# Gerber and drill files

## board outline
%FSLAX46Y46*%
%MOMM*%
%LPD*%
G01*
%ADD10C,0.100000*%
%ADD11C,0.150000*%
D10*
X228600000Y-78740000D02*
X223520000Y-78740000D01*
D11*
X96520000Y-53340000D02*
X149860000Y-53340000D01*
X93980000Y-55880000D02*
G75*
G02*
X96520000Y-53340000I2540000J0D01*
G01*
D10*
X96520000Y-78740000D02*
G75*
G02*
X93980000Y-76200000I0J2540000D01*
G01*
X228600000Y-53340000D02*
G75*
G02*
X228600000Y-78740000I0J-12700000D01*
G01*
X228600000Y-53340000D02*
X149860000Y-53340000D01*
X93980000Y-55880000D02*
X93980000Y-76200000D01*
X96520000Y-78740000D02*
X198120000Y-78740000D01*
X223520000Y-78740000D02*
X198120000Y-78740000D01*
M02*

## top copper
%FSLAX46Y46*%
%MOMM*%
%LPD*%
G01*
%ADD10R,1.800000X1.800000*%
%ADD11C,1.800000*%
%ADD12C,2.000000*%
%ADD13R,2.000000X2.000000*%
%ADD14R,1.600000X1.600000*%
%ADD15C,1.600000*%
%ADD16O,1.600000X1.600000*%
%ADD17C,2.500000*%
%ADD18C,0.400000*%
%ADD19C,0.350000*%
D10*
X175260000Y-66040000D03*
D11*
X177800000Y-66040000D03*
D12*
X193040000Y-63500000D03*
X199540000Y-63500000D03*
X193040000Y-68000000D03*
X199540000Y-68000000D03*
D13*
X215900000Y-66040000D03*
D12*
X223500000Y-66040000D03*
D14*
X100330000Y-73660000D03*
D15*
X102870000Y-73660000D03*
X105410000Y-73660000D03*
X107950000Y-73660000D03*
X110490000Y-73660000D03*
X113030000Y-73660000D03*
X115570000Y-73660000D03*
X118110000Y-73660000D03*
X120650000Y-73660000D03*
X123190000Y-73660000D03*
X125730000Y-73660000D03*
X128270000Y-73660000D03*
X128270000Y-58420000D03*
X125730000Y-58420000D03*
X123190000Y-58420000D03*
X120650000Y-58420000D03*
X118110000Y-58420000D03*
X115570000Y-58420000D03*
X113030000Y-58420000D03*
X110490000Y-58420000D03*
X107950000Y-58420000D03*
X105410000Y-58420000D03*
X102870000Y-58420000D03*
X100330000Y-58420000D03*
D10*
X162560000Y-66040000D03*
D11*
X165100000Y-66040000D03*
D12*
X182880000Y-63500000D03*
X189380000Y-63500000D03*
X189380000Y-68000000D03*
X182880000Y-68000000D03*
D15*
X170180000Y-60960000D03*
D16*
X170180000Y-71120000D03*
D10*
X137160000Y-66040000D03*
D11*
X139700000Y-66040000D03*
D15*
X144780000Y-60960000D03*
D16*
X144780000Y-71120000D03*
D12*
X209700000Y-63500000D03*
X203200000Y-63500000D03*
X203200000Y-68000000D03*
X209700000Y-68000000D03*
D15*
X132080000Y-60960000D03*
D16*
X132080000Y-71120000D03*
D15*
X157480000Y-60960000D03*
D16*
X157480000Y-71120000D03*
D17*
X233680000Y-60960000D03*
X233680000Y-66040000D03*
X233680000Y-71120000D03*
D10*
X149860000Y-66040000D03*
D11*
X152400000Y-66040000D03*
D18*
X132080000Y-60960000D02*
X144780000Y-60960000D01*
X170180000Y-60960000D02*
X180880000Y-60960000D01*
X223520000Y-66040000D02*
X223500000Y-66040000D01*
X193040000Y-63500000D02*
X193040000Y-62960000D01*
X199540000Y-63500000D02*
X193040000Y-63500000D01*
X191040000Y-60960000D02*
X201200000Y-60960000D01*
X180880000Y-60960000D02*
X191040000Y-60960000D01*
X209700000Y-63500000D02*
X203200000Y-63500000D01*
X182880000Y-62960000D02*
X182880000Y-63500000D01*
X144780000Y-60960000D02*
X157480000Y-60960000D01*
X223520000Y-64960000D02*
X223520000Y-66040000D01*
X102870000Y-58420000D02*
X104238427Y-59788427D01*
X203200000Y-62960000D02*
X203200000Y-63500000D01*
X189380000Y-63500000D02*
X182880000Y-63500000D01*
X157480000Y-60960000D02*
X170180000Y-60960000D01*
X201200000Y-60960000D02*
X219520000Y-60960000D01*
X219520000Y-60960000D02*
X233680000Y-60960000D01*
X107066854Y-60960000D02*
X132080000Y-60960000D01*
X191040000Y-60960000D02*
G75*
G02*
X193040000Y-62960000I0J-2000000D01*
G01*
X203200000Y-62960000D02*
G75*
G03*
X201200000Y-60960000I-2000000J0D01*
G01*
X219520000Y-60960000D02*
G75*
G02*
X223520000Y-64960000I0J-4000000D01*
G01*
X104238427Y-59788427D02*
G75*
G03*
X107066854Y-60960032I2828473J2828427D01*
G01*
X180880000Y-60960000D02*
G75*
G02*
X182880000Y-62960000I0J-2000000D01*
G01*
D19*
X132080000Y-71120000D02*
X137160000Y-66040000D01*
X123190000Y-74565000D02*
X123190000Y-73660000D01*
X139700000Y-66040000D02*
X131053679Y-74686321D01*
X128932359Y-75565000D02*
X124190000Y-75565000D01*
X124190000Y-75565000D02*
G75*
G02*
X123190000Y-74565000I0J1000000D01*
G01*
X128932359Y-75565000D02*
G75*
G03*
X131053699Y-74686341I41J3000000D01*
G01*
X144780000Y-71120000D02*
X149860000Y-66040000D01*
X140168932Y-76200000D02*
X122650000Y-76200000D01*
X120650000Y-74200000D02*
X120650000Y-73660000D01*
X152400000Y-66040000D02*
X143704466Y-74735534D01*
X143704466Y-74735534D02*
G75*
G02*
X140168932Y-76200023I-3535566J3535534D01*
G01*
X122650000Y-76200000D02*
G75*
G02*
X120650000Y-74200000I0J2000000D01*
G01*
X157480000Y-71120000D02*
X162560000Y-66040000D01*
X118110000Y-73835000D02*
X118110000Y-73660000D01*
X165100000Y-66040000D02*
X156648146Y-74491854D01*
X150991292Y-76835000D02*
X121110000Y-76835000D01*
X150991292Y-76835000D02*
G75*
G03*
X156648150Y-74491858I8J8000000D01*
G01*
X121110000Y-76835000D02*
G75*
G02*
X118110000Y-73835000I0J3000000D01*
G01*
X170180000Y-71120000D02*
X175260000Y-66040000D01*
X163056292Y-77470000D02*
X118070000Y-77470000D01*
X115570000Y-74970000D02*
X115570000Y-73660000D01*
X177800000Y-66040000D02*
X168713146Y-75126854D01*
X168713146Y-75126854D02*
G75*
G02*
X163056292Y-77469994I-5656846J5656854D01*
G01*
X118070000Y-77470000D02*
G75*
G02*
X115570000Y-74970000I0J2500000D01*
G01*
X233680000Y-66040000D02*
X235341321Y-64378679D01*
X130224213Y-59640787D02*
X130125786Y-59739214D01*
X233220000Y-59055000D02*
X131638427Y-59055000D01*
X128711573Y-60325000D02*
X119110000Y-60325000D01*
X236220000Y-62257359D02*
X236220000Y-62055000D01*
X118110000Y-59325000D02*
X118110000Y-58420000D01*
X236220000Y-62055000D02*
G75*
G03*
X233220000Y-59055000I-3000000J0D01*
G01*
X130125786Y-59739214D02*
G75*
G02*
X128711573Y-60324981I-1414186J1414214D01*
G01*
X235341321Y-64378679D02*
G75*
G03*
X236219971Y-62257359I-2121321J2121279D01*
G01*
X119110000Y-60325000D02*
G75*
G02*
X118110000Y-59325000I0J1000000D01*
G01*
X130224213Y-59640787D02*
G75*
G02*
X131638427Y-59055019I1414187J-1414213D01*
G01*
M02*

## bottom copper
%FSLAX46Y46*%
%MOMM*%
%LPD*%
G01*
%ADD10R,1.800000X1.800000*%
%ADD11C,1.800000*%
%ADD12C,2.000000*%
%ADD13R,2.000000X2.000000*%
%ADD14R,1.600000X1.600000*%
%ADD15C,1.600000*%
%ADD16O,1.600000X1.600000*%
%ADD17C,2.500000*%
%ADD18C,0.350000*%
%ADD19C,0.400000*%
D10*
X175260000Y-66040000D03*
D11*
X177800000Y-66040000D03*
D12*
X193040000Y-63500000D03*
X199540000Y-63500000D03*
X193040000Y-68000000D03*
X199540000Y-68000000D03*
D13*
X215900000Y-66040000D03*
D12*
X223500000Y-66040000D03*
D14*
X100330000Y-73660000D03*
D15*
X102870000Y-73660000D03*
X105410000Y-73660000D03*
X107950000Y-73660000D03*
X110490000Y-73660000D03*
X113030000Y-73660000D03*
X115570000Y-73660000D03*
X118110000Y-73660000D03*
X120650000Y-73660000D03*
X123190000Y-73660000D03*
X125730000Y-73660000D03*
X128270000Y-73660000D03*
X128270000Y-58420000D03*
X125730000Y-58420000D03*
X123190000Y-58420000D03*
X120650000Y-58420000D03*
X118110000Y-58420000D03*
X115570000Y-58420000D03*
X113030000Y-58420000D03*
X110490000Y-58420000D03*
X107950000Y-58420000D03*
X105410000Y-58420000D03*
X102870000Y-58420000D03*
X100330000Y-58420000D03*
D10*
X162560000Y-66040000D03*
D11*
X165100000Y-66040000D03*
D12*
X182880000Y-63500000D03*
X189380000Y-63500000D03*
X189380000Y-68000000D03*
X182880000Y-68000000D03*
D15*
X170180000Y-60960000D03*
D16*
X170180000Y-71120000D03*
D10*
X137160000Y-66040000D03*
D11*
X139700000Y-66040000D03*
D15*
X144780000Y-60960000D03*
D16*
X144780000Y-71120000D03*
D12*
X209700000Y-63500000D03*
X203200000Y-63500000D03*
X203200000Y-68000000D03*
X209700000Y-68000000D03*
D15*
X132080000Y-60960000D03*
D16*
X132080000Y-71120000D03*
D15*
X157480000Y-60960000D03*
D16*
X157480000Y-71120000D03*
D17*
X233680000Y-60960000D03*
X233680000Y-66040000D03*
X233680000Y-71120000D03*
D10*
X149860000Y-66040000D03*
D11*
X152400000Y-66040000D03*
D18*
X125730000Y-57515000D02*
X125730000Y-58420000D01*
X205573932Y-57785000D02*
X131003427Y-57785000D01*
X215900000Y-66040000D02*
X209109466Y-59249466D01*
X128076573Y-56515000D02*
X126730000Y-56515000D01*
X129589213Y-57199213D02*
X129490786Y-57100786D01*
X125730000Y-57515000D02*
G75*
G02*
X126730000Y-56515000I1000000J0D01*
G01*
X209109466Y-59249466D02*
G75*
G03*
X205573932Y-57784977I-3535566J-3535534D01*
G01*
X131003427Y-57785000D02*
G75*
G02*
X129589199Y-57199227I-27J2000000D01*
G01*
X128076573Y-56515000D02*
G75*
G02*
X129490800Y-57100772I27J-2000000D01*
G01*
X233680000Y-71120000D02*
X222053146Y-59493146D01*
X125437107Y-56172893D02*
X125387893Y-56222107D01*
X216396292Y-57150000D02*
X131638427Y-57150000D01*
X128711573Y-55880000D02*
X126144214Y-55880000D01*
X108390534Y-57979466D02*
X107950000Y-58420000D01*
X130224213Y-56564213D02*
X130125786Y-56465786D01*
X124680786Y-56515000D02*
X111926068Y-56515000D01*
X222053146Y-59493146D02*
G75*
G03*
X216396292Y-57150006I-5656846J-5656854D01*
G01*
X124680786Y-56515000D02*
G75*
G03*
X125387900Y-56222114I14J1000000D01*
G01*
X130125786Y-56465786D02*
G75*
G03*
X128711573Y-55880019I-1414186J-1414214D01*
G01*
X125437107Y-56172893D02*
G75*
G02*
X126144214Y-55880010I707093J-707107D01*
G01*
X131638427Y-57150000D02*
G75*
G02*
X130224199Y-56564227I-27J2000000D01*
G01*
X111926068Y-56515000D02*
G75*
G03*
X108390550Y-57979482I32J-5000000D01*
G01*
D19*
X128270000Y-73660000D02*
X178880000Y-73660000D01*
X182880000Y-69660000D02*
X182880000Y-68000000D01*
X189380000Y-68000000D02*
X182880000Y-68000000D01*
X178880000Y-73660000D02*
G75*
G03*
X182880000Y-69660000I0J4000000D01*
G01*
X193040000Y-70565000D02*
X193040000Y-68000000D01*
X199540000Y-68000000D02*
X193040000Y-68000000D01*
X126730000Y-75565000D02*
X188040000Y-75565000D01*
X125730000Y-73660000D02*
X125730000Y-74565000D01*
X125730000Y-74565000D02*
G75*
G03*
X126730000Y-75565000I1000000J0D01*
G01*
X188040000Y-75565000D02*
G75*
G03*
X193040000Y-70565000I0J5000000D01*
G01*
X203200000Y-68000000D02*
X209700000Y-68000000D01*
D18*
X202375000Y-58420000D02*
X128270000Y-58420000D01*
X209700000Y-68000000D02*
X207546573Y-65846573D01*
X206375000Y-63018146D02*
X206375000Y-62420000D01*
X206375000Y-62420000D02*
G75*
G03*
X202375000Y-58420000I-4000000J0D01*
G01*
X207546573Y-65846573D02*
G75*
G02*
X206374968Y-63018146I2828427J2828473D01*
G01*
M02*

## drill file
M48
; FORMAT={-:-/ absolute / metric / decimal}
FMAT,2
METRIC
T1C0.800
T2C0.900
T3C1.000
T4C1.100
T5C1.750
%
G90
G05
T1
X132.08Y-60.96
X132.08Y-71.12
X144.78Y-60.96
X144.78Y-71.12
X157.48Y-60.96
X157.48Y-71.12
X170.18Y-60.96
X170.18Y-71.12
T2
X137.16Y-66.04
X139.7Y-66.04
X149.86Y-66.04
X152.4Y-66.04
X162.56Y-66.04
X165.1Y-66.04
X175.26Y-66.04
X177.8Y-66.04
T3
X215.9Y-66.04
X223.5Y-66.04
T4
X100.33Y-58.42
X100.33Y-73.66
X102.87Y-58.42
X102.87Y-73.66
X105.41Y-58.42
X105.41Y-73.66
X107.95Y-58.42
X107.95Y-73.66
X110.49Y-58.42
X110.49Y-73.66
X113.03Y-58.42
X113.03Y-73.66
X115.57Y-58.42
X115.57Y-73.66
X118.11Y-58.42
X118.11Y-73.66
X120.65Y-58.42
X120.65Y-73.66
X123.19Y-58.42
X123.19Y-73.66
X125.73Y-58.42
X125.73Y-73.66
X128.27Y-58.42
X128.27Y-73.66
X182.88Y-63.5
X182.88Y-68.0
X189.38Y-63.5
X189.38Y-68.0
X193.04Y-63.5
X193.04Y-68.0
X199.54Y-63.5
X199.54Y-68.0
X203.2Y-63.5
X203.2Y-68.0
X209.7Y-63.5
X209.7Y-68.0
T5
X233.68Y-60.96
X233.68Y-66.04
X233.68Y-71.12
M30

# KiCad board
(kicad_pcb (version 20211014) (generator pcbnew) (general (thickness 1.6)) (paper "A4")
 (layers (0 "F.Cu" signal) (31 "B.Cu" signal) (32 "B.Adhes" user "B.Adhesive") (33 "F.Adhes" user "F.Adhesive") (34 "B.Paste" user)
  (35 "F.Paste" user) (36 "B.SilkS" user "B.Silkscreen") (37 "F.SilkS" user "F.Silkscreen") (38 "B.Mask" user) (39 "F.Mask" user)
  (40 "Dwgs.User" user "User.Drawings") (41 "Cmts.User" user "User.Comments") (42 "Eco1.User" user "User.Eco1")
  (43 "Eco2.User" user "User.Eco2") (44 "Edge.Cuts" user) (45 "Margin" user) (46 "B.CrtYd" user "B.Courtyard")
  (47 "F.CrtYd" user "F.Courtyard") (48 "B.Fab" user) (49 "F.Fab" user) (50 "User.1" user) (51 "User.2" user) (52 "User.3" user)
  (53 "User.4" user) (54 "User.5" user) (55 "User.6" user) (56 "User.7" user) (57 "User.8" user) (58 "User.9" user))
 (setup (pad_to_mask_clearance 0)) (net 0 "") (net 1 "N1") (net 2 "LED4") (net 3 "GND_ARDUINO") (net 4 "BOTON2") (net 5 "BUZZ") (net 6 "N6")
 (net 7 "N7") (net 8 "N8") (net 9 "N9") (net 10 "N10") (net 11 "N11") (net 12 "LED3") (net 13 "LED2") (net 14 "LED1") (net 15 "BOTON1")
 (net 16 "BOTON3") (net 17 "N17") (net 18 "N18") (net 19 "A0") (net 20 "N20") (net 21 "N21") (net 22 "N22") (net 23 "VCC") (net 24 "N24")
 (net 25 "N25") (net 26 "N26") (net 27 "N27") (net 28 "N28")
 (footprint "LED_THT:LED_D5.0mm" (layer "F.Cu") (at 175.26 66.04)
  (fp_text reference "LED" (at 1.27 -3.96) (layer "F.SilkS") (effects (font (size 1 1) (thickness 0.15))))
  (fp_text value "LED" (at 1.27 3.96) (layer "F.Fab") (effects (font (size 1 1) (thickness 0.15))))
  (pad "1" thru_hole rect (at 0 0) (size 1.8 1.8) (drill 0.9) (layers *.Cu *.Mask) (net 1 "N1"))
  (pad "2" thru_hole circle (at 2.54 0) (size 1.8 1.8) (drill 0.9) (layers *.Cu *.Mask) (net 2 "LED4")))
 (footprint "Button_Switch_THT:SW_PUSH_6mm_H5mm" (layer "F.Cu") (at 193.04 63.5)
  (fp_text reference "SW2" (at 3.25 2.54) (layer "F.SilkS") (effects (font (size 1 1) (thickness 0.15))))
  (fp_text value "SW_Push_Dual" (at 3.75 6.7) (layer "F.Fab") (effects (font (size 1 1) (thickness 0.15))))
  (pad "1" thru_hole circle (at 0 0 90) (size 2 2) (drill 1.1) (layers *.Cu *.Mask) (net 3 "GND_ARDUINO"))
  (pad "1" thru_hole circle (at 6.5 0 90) (size 2 2) (drill 1.1) (layers *.Cu *.Mask) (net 3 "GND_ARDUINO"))
  (pad "2" thru_hole circle (at 0 4.5 90) (size 2 2) (drill 1.1) (layers *.Cu *.Mask) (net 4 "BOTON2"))
  (pad "2" thru_hole circle (at 6.5 4.5 90) (size 2 2) (drill 1.1) (layers *.Cu *.Mask) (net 4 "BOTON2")))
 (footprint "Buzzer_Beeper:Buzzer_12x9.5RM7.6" (layer "F.Cu") (at 215.9 66.04)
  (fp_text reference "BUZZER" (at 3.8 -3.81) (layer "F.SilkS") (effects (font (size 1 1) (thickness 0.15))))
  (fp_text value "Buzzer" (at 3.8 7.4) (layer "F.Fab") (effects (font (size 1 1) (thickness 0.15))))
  (pad "1" thru_hole rect (at 0 0) (size 2 2) (drill 1) (layers *.Cu *.Mask) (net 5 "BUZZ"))
  (pad "2" thru_hole circle (at 7.6 0) (size 2 2) (drill 1) (layers *.Cu *.Mask) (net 3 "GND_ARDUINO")))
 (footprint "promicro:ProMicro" (layer "F.Cu") (at 114.3 66.04)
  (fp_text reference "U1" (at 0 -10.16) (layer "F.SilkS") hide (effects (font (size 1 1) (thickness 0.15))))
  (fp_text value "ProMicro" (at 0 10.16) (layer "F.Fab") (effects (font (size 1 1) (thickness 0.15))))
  (pad "1" thru_hole rect locked (at -13.97 7.62) (size 1.6 1.6) (drill 1.1) (layers *.Cu *.Mask "F.SilkS") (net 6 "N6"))
  (pad "2" thru_hole circle locked (at -11.43 7.62) (size 1.6 1.6) (drill 1.1) (layers *.Cu *.Mask "F.SilkS") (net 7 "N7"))
  (pad "3" thru_hole circle locked (at -8.89 7.62) (size 1.6 1.6) (drill 1.1) (layers *.Cu *.Mask "F.SilkS") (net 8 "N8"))
  (pad "4" thru_hole circle locked (at -6.35 7.62) (size 1.6 1.6) (drill 1.1) (layers *.Cu *.Mask "F.SilkS") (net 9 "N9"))
  (pad "5" thru_hole circle locked (at -3.81 7.62) (size 1.6 1.6) (drill 1.1) (layers *.Cu *.Mask "F.SilkS") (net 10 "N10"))
  (pad "6" thru_hole circle locked (at -1.27 7.62) (size 1.6 1.6) (drill 1.1) (layers *.Cu *.Mask "F.SilkS") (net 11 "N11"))
  (pad "7" thru_hole circle locked (at 1.27 7.62) (size 1.6 1.6) (drill 1.1) (layers *.Cu *.Mask "F.SilkS") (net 2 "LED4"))
  (pad "8" thru_hole circle locked (at 3.81 7.62) (size 1.6 1.6) (drill 1.1) (layers *.Cu *.Mask "F.SilkS") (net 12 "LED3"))
  (pad "9" thru_hole circle locked (at 6.35 7.62) (size 1.6 1.6) (drill 1.1) (layers *.Cu *.Mask "F.SilkS") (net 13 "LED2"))
  (pad "10" thru_hole circle locked (at 8.89 7.62) (size 1.6 1.6) (drill 1.1) (layers *.Cu *.Mask "F.SilkS") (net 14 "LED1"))
  (pad "11" thru_hole circle locked (at 11.43 7.62) (size 1.6 1.6) (drill 1.1) (layers *.Cu *.Mask "F.SilkS") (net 4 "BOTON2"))
  (pad "12" thru_hole circle locked (at 13.97 7.62) (size 1.6 1.6) (drill 1.1) (layers *.Cu *.Mask "F.SilkS") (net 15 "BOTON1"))
  (pad "13" thru_hole circle locked (at 13.97 -7.62) (size 1.6 1.6) (drill 1.1) (layers *.Cu *.Mask "F.SilkS") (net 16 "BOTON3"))
  (pad "14" thru_hole circle locked (at 11.43 -7.62) (size 1.6 1.6) (drill 1.1) (layers *.Cu *.Mask "F.SilkS") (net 5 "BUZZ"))
  (pad "15" thru_hole circle locked (at 8.89 -7.62) (size 1.6 1.6) (drill 1.1) (layers *.Cu *.Mask "F.SilkS") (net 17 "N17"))
  (pad "16" thru_hole circle locked (at 6.35 -7.62) (size 1.6 1.6) (drill 1.1) (layers *.Cu *.Mask "F.SilkS") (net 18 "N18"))
  (pad "17" thru_hole circle locked (at 3.81 -7.62) (size 1.6 1.6) (drill 1.1) (layers *.Cu *.Mask "F.SilkS") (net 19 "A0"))
  (pad "18" thru_hole circle locked (at 1.27 -7.62) (size 1.6 1.6) (drill 1.1) (layers *.Cu *.Mask "F.SilkS") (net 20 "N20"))
  (pad "19" thru_hole circle locked (at -1.27 -7.62) (size 1.6 1.6) (drill 1.1) (layers *.Cu *.Mask "F.SilkS") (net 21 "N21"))
  (pad "20" thru_hole circle locked (at -3.81 -7.62) (size 1.6 1.6) (drill 1.1) (layers *.Cu *.Mask "F.SilkS") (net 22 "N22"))
  (pad "21" thru_hole circle locked (at -6.35 -7.62) (size 1.6 1.6) (drill 1.1) (layers *.Cu *.Mask "F.SilkS") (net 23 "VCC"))
  (pad "22" thru_hole circle locked (at -8.89 -7.62) (size 1.6 1.6) (drill 1.1) (layers *.Cu *.Mask "F.SilkS") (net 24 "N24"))
  (pad "23" thru_hole circle locked (at -11.43 -7.62) (size 1.6 1.6) (drill 1.1) (layers *.Cu *.Mask "F.SilkS") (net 3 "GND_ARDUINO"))
  (pad "24" thru_hole circle locked (at -13.97 -7.62) (size 1.6 1.6) (drill 1.1) (layers *.Cu *.Mask "F.SilkS") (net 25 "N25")))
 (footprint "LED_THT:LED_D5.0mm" (layer "F.Cu") (at 162.56 66.04)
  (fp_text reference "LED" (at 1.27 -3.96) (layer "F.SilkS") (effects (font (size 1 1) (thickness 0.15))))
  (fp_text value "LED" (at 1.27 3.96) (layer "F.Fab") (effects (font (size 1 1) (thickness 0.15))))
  (pad "1" thru_hole rect (at 0 0) (size 1.8 1.8) (drill 0.9) (layers *.Cu *.Mask) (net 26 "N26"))
  (pad "2" thru_hole circle (at 2.54 0) (size 1.8 1.8) (drill 0.9) (layers *.Cu *.Mask) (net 12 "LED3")))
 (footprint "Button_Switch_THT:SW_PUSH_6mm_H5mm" (layer "F.Cu") (at 182.88 63.5)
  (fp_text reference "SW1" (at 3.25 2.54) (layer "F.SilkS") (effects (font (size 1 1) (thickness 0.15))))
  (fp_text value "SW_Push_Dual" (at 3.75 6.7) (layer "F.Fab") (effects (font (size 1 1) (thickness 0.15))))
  (pad "1" thru_hole circle (at 0 0 90) (size 2 2) (drill 1.1) (layers *.Cu *.Mask) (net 3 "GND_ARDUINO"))
  (pad "1" thru_hole circle (at 6.5 0 90) (size 2 2) (drill 1.1) (layers *.Cu *.Mask) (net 3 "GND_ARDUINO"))
  (pad "2" thru_hole circle (at 6.5 4.5 90) (size 2 2) (drill 1.1) (layers *.Cu *.Mask) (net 15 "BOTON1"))
  (pad "2" thru_hole circle (at 0 4.5 90) (size 2 2) (drill 1.1) (layers *.Cu *.Mask) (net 15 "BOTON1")))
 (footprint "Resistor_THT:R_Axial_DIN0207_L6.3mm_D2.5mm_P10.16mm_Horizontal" (layer "F.Cu") (at 170.18 60.96 -90)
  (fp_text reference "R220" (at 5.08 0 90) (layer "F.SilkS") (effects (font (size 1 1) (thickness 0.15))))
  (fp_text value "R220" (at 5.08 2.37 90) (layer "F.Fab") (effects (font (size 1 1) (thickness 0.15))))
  (pad "1" thru_hole circle (at 0 0 270) (size 1.6 1.6) (drill 0.8) (layers *.Cu *.Mask) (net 3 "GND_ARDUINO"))
  (pad "2" thru_hole oval (at 10.16 0 270) (size 1.6 1.6) (drill 0.8) (layers *.Cu *.Mask) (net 1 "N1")))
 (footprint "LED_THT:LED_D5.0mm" (layer "F.Cu") (at 137.16 66.04)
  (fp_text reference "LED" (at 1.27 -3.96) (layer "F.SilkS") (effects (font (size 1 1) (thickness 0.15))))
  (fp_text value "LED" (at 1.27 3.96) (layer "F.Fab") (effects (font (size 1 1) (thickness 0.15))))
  (pad "1" thru_hole rect (at 0 0) (size 1.8 1.8) (drill 0.9) (layers *.Cu *.Mask) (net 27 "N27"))
  (pad "2" thru_hole circle (at 2.54 0) (size 1.8 1.8) (drill 0.9) (layers *.Cu *.Mask) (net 14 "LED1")))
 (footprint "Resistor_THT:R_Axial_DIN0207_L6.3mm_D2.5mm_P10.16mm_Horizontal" (layer "F.Cu") (at 144.78 60.96 -90)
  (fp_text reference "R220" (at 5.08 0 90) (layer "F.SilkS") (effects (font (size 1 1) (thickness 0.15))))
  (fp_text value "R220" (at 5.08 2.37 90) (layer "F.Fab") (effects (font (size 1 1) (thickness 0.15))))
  (pad "1" thru_hole circle (at 0 0 270) (size 1.6 1.6) (drill 0.8) (layers *.Cu *.Mask) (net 3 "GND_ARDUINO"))
  (pad "2" thru_hole oval (at 10.16 0 270) (size 1.6 1.6) (drill 0.8) (layers *.Cu *.Mask) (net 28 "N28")))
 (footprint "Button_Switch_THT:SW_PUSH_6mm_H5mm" (layer "F.Cu") (at 203.2 63.5)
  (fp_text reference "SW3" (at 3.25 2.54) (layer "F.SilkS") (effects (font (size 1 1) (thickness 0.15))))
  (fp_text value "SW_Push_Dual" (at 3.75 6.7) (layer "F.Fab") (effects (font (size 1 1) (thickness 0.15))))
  (pad "1" thru_hole circle (at 6.5 0 90) (size 2 2) (drill 1.1) (layers *.Cu *.Mask) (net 3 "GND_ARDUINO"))
  (pad "1" thru_hole circle (at 0 0 90) (size 2 2) (drill 1.1) (layers *.Cu *.Mask) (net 3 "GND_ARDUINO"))
  (pad "2" thru_hole circle (at 0 4.5 90) (size 2 2) (drill 1.1) (layers *.Cu *.Mask) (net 16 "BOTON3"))
  (pad "2" thru_hole circle (at 6.5 4.5 90) (size 2 2) (drill 1.1) (layers *.Cu *.Mask) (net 16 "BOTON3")))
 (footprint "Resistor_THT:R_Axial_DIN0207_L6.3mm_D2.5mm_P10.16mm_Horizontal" (layer "F.Cu") (at 132.08 60.96 -90)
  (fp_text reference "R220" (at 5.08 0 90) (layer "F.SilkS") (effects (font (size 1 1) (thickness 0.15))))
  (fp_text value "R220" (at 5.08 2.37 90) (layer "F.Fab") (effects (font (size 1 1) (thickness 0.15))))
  (pad "1" thru_hole circle (at 0 0 270) (size 1.6 1.6) (drill 0.8) (layers *.Cu *.Mask) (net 3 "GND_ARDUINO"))
  (pad "2" thru_hole oval (at 10.16 0 270) (size 1.6 1.6) (drill 0.8) (layers *.Cu *.Mask) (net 27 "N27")))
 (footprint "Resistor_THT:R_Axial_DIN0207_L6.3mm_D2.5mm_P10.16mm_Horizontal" (layer "F.Cu") (at 157.48 60.96 -90)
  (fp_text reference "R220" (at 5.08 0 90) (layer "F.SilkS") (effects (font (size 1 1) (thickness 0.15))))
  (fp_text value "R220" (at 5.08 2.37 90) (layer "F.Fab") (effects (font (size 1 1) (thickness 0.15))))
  (pad "1" thru_hole circle (at 0 0 270) (size 1.6 1.6) (drill 0.8) (layers *.Cu *.Mask) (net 3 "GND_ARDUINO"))
  (pad "2" thru_hole oval (at 10.16 0 270) (size 1.6 1.6) (drill 0.8) (layers *.Cu *.Mask) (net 26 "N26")))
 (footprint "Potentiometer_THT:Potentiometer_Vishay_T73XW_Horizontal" (layer "F.Cu") (at 233.68 63.5)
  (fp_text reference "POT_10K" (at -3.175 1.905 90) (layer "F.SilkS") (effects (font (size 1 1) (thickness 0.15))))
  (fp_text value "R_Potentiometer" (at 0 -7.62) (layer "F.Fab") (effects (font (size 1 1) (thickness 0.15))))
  (pad "1" thru_hole circle (at 0 -2.54) (size 2.5 2.5) (drill 1.75) (layers *.Cu *.Mask) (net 3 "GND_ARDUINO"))
  (pad "2" thru_hole circle (at 0 2.54) (size 2.5 2.5) (drill 1.75) (layers *.Cu *.Mask) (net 19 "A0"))
  (pad "3" thru_hole circle (at 0 7.62) (size 2.5 2.5) (drill 1.75) (layers *.Cu *.Mask) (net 23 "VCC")))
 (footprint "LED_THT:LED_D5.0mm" (layer "F.Cu") (at 149.86 66.04)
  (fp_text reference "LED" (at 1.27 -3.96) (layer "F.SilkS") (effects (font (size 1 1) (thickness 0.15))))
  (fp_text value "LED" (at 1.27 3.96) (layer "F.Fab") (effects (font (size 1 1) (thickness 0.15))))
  (pad "1" thru_hole rect (at 0 0) (size 1.8 1.8) (drill 0.9) (layers *.Cu *.Mask) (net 28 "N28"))
  (pad "2" thru_hole circle (at 2.54 0) (size 1.8 1.8) (drill 0.9) (layers *.Cu *.Mask) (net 13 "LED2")))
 (gr_line (start 228.6 78.74) (end 223.52 78.74) (layer "Edge.Cuts") (width 0.1))
 (gr_line (start 96.52 53.34) (end 149.86 53.34) (layer "Edge.Cuts") (width 0.15))
 (gr_arc (start 93.98 55.88) (mid 94.723949 54.083949) (end 96.52 53.34) (layer "Edge.Cuts") (width 0.15))
 (gr_arc (start 96.52 78.74) (mid 94.723949 77.996051) (end 93.98 76.2) (layer "Edge.Cuts") (width 0.1))
 (gr_arc (start 228.6 53.34) (mid 241.3 66.04) (end 228.6 78.74) (layer "Edge.Cuts") (width 0.1))
 (gr_line (start 228.6 53.34) (end 149.86 53.34) (layer "Edge.Cuts") (width 0.1))
 (gr_line (start 93.98 55.88) (end 93.98 76.2) (layer "Edge.Cuts") (width 0.1))
 (gr_line (start 96.52 78.74) (end 198.12 78.74) (layer "Edge.Cuts") (width 0.1))
 (gr_line (start 223.52 78.74) (end 198.12 78.74) (layer "Edge.Cuts") (width 0.1))
 (segment (start 125.73 57.515) (end 125.73 58.42) (width 0.35) (layer "B.Cu") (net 5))
 (segment (start 205.573932 57.785) (end 131.003427 57.785) (width 0.35) (layer "B.Cu") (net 5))
 (segment (start 215.9 66.04) (end 209.109466 59.249466) (width 0.35) (layer "B.Cu") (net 5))
 (segment (start 128.076573 56.515) (end 126.73 56.515) (width 0.35) (layer "B.Cu") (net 5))
 (segment (start 129.589213 57.199213) (end 129.490786 57.100786) (width 0.35) (layer "B.Cu") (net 5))
 (arc (start 125.73 57.515) (mid 126.022893 56.807893) (end 126.73 56.515) (width 0.35) (layer "B.Cu") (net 5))
 (arc (start 209.109466 59.249466) (mid 207.487349 58.165602) (end 205.573932 57.785) (width 0.35) (layer "B.Cu") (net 5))
 (arc (start 131.003427 57.785) (mid 130.23806 57.632759) (end 129.589213 57.199213) (width 0.35) (layer "B.Cu") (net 5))
 (arc (start 128.076573 56.515) (mid 128.84194 56.667241) (end 129.490786 57.100786) (width 0.35) (layer "B.Cu") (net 5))
 (segment (start 132.08 60.96) (end 144.78 60.96) (width 0.4) (layer "F.Cu") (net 3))
 (segment (start 170.18 60.96) (end 180.88 60.96) (width 0.4) (layer "F.Cu") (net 3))
 (segment (start 223.52 66.04) (end 223.5 66.04) (width 0.4) (layer "F.Cu") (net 3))
 (segment (start 193.04 63.5) (end 193.04 62.96) (width 0.4) (layer "F.Cu") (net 3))
 (segment (start 199.54 63.5) (end 193.04 63.5) (width 0.4) (layer "F.Cu") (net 3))
 (segment (start 191.04 60.96) (end 201.2 60.96) (width 0.4) (layer "F.Cu") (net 3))
 (segment (start 180.88 60.96) (end 191.04 60.96) (width 0.4) (layer "F.Cu") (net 3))
 (segment (start 209.7 63.5) (end 203.2 63.5) (width 0.4) (layer "F.Cu") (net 3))
 (segment (start 182.88 62.96) (end 182.88 63.5) (width 0.4) (layer "F.Cu") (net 3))
 (segment (start 144.78 60.96) (end 157.48 60.96) (width 0.4) (layer "F.Cu") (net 3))
 (segment (start 223.52 64.96) (end 223.52 66.04) (width 0.4) (layer "F.Cu") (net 3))
 (segment (start 102.87 58.42) (end 104.238427 59.788427) (width 0.4) (layer "F.Cu") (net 3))
 (segment (start 203.2 62.96) (end 203.2 63.5) (width 0.4) (layer "F.Cu") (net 3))
 (segment (start 189.38 63.5) (end 182.88 63.5) (width 0.4) (layer "F.Cu") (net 3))
 (segment (start 157.48 60.96) (end 170.18 60.96) (width 0.4) (layer "F.Cu") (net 3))
 (segment (start 201.2 60.96) (end 219.52 60.96) (width 0.4) (layer "F.Cu") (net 3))
 (segment (start 219.52 60.96) (end 233.68 60.96) (width 0.4) (layer "F.Cu") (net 3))
 (segment (start 107.066854 60.96) (end 132.08 60.96) (width 0.4) (layer "F.Cu") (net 3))
 (arc (start 191.04 60.96) (mid 192.454214 61.545786) (end 193.04 62.96) (width 0.4) (layer "F.Cu") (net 3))
 (arc (start 203.2 62.96) (mid 202.614214 61.545786) (end 201.2 60.96) (width 0.4) (layer "F.Cu") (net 3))
 (arc (start 219.52 60.96) (mid 222.348427 62.131573) (end 223.52 64.96) (width 0.4) (layer "F.Cu") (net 3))
 (arc (start 104.238427 59.788427) (mid 105.53612 60.655518) (end 107.066854 60.96) (width 0.4) (layer "F.Cu") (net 3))
 (arc (start 180.88 60.96) (mid 182.294214 61.545786) (end 182.88 62.96) (width 0.4) (layer "F.Cu") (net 3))
 (segment (start 132.08 71.12) (end 137.16 66.04) (width 0.35) (layer "F.Cu") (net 27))
 (segment (start 123.19 74.565) (end 123.19 73.66) (width 0.35) (layer "F.Cu") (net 14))
 (segment (start 139.7 66.04) (end 131.053679 74.686321) (width 0.35) (layer "F.Cu") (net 14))
 (segment (start 128.932359 75.565) (end 124.19 75.565) (width 0.35) (layer "F.Cu") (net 14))
 (arc (start 124.19 75.565) (mid 123.482893 75.272107) (end 123.19 74.565) (width 0.35) (layer "F.Cu") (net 14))
 (arc (start 128.932359 75.565) (mid 130.080409 75.336639) (end 131.053679 74.686321) (width 0.35) (layer "F.Cu") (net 14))
 (segment (start 144.78 71.12) (end 149.86 66.04) (width 0.35) (layer "F.Cu") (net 28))
 (segment (start 140.168932 76.2) (end 122.65 76.2) (width 0.35) (layer "F.Cu") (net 13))
 (segment (start 120.65 74.2) (end 120.65 73.66) (width 0.35) (layer "F.Cu") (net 13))
 (segment (start 152.4 66.04) (end 143.704466 74.735534) (width 0.35) (layer "F.Cu") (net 13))
 (arc (start 143.704466 74.735534) (mid 142.082349 75.819398) (end 140.168932 76.2) (width 0.35) (layer "F.Cu") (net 13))
 (arc (start 122.65 76.2) (mid 121.235786 75.614214) (end 120.65 74.2) (width 0.35) (layer "F.Cu") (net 13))
 (segment (start 157.48 71.12) (end 162.56 66.04) (width 0.35) (layer "F.Cu") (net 26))
 (segment (start 118.11 73.835) (end 118.11 73.66) (width 0.35) (layer "F.Cu") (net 12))
 (segment (start 165.1 66.04) (end 156.648146 74.491854) (width 0.35) (layer "F.Cu") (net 12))
 (segment (start 150.991292 76.835) (end 121.11 76.835) (width 0.35) (layer "F.Cu") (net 12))
 (arc (start 150.991292 76.835) (mid 154.052759 76.226036) (end 156.648146 74.491854) (width 0.35) (layer "F.Cu") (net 12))
 (arc (start 121.11 76.835) (mid 118.98868 75.95632) (end 118.11 73.835) (width 0.35) (layer "F.Cu") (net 12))
 (segment (start 170.18 71.12) (end 175.26 66.04) (width 0.35) (layer "F.Cu") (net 1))
 (segment (start 163.056292 77.47) (end 118.07 77.47) (width 0.35) (layer "F.Cu") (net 2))
 (segment (start 115.57 74.97) (end 115.57 73.66) (width 0.35) (layer "F.Cu") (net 2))
 (segment (start 177.8 66.04) (end 168.713146 75.126854) (width 0.35) (layer "F.Cu") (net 2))
 (arc (start 168.713146 75.126854) (mid 166.117759 76.861036) (end 163.056292 77.47) (width 0.35) (layer "F.Cu") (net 2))
 (arc (start 118.07 77.47) (mid 116.302233 76.737767) (end 115.57 74.97) (width 0.35) (layer "F.Cu") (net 2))
 (segment (start 233.68 66.04) (end 235.341321 64.378679) (width 0.35) (layer "F.Cu") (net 19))
 (segment (start 130.224213 59.640787) (end 130.125786 59.739214) (width 0.35) (layer "F.Cu") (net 19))
 (segment (start 233.22 59.055) (end 131.638427 59.055) (width 0.35) (layer "F.Cu") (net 19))
 (segment (start 128.711573 60.325) (end 119.11 60.325) (width 0.35) (layer "F.Cu") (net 19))
 (segment (start 236.22 62.257359) (end 236.22 62.055) (width 0.35) (layer "F.Cu") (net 19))
 (segment (start 118.11 59.325) (end 118.11 58.42) (width 0.35) (layer "F.Cu") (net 19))
 (arc (start 236.22 62.055) (mid 235.34132 59.93368) (end 233.22 59.055) (width 0.35) (layer "F.Cu") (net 19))
 (arc (start 130.125786 59.739214) (mid 129.47694 60.172759) (end 128.711573 60.325) (width 0.35) (layer "F.Cu") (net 19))
 (arc (start 235.341321 64.378679) (mid 235.991639 63.405409) (end 236.22 62.257359) (width 0.35) (layer "F.Cu") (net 19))
 (arc (start 119.11 60.325) (mid 118.402893 60.032107) (end 118.11 59.325) (width 0.35) (layer "F.Cu") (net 19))
 (arc (start 130.224213 59.640787) (mid 130.87306 59.207241) (end 131.638427 59.055) (width 0.35) (layer "F.Cu") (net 19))
 (segment (start 233.68 71.12) (end 222.053146 59.493146) (width 0.35) (layer "B.Cu") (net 23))
 (segment (start 125.437107 56.172893) (end 125.387893 56.222107) (width 0.35) (layer "B.Cu") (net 23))
 (segment (start 216.396292 57.15) (end 131.638427 57.15) (width 0.35) (layer "B.Cu") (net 23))
 (segment (start 128.711573 55.88) (end 126.144214 55.88) (width 0.35) (layer "B.Cu") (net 23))
 (segment (start 108.390534 57.979466) (end 107.95 58.42) (width 0.35) (layer "B.Cu") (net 23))
 (segment (start 130.224213 56.564213) (end 130.125786 56.465786) (width 0.35) (layer "B.Cu") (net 23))
 (segment (start 124.680786 56.515) (end 111.926068 56.515) (width 0.35) (layer "B.Cu") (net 23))
 (arc (start 222.053146 59.493146) (mid 219.457759 57.758964) (end 216.396292 57.15) (width 0.35) (layer "B.Cu") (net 23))
 (arc (start 124.680786 56.515) (mid 125.063469 56.43888) (end 125.387893 56.222107) (width 0.35) (layer "B.Cu") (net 23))
 (arc (start 130.125786 56.465786) (mid 129.47694 56.032241) (end 128.711573 55.88) (width 0.35) (layer "B.Cu") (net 23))
 (arc (start 125.437107 56.172893) (mid 125.76153 55.95612) (end 126.144214 55.88) (width 0.35) (layer "B.Cu") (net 23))
 (arc (start 131.638427 57.15) (mid 130.87306 56.997759) (end 130.224213 56.564213) (width 0.35) (layer "B.Cu") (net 23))
 (arc (start 111.926068 56.515) (mid 110.012651 56.895602) (end 108.390534 57.979466) (width 0.35) (layer "B.Cu") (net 23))
 (segment (start 128.27 73.66) (end 178.88 73.66) (width 0.4) (layer "B.Cu") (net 15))
 (segment (start 182.88 69.66) (end 182.88 68) (width 0.4) (layer "B.Cu") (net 15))
 (segment (start 189.38 68) (end 182.88 68) (width 0.4) (layer "B.Cu") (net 15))
 (arc (start 178.88 73.66) (mid 181.708427 72.488427) (end 182.88 69.66) (width 0.4) (layer "B.Cu") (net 15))
 (segment (start 193.04 70.565) (end 193.04 68) (width 0.4) (layer "B.Cu") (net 4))
 (segment (start 199.54 68) (end 193.04 68) (width 0.4) (layer "B.Cu") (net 4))
 (segment (start 126.73 75.565) (end 188.04 75.565) (width 0.4) (layer "B.Cu") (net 4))
 (segment (start 125.73 73.66) (end 125.73 74.565) (width 0.4) (layer "B.Cu") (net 4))
 (arc (start 125.73 74.565) (mid 126.022893 75.272107) (end 126.73 75.565) (width 0.4) (layer "B.Cu") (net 4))
 (arc (start 188.04 75.565) (mid 191.575534 74.100534) (end 193.04 70.565) (width 0.4) (layer "B.Cu") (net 4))
 (segment (start 203.2 68) (end 209.7 68) (width 0.4) (layer "B.Cu") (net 16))
 (segment (start 202.375 58.42) (end 128.27 58.42) (width 0.35) (layer "B.Cu") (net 16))
 (segment (start 209.7 68) (end 207.546573 65.846573) (width 0.35) (layer "B.Cu") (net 16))
 (segment (start 206.375 63.018146) (end 206.375 62.42) (width 0.35) (layer "B.Cu") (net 16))
 (arc (start 206.375 62.42) (mid 205.203427 59.591573) (end 202.375 58.42) (width 0.35) (layer "B.Cu") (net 16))
 (arc (start 207.546573 65.846573) (mid 206.679482 64.54888) (end 206.375 63.018146) (width 0.35) (layer "B.Cu") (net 16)))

